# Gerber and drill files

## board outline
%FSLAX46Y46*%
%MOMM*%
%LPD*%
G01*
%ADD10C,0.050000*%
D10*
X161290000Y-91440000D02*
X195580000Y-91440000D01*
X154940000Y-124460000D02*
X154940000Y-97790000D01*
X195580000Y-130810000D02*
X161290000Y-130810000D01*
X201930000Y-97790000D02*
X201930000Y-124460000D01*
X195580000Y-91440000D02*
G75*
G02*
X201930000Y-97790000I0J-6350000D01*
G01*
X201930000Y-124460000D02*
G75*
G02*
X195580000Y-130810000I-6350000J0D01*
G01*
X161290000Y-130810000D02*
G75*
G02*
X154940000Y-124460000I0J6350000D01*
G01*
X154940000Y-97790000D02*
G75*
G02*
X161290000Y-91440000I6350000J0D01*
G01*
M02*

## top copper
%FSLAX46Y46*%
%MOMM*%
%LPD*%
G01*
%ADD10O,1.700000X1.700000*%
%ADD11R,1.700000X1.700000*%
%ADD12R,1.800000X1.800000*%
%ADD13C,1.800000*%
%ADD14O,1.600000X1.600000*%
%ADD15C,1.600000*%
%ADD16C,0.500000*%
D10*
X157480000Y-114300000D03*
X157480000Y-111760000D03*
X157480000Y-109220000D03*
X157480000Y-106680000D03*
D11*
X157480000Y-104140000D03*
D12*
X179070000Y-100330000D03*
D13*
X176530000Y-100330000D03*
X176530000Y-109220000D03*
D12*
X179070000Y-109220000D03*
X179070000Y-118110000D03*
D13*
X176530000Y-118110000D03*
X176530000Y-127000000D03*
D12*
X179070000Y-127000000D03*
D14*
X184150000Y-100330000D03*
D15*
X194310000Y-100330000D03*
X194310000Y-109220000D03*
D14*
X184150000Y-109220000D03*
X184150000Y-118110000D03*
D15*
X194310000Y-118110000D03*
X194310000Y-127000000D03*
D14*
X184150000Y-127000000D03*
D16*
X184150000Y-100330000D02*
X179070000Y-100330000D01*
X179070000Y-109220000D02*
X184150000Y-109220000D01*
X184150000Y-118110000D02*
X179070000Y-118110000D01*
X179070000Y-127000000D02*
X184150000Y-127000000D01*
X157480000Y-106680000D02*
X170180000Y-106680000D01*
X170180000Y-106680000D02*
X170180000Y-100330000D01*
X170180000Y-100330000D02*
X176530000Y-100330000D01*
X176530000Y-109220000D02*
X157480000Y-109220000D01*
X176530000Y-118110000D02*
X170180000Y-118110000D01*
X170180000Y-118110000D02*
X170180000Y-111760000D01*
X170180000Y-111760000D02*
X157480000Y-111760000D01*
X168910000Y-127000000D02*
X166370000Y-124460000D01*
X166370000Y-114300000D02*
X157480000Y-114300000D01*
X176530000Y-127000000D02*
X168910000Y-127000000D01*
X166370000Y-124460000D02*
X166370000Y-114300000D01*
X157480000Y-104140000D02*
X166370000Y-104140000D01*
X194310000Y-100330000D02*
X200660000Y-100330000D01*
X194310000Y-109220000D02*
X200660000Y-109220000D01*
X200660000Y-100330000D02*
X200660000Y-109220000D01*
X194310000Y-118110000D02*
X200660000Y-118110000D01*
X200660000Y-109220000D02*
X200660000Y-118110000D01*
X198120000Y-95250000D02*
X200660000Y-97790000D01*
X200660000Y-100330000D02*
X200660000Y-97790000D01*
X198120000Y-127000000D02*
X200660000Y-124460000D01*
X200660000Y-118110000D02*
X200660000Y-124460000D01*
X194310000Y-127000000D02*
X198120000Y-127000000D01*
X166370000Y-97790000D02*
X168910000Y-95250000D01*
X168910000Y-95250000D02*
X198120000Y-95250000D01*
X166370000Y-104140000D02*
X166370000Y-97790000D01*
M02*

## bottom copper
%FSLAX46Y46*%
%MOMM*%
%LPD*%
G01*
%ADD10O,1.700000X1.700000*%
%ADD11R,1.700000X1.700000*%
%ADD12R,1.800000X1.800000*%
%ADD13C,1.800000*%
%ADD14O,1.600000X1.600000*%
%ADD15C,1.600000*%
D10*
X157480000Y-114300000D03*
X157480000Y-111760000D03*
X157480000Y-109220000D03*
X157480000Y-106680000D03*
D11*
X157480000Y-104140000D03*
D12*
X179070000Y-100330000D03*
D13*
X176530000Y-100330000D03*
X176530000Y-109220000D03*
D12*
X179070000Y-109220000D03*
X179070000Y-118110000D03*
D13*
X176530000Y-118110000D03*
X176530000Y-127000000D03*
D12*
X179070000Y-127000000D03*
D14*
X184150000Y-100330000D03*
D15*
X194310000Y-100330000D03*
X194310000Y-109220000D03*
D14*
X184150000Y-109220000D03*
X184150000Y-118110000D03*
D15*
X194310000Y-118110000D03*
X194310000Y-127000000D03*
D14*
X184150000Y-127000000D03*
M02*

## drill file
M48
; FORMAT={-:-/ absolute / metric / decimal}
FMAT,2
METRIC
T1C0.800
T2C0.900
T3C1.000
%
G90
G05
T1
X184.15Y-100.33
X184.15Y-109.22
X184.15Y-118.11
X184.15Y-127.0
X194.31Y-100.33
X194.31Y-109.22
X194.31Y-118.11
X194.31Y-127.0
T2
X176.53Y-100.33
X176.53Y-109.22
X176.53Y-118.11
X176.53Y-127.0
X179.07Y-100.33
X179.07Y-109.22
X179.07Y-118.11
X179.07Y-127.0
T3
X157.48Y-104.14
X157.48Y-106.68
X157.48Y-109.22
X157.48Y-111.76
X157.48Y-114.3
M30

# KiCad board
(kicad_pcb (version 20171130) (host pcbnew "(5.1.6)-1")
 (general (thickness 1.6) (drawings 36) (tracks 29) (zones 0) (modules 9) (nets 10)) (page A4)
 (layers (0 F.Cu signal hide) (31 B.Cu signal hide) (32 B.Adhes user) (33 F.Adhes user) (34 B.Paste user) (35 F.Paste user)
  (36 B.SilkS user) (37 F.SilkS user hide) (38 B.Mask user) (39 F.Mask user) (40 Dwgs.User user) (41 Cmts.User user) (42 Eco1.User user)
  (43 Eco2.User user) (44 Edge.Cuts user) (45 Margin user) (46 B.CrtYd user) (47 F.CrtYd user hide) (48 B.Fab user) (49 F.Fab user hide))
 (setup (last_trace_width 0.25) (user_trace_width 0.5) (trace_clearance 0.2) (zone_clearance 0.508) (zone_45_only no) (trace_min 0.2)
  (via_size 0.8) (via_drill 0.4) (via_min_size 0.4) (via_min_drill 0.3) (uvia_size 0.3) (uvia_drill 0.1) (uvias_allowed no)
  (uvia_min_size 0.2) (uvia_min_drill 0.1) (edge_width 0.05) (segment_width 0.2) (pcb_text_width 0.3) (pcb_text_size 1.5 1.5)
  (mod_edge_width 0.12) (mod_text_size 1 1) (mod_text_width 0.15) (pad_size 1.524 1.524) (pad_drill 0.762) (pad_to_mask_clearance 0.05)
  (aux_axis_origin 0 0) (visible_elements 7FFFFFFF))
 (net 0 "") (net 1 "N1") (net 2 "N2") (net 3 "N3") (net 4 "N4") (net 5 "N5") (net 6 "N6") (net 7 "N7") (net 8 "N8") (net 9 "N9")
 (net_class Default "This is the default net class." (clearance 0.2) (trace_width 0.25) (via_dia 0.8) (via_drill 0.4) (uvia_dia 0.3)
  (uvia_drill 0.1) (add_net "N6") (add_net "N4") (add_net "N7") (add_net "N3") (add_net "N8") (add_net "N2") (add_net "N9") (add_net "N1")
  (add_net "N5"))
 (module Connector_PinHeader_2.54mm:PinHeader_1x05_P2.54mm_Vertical (layer F.Cu) (at 157.48 104.14)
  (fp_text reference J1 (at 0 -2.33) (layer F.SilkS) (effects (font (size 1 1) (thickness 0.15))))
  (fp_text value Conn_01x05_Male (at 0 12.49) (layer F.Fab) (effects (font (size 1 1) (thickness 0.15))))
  (pad 5 thru_hole oval (at 0 10.16) (size 1.7 1.7) (drill 1) (layers *.Cu *.Mask) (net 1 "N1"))
  (pad 4 thru_hole oval (at 0 7.62) (size 1.7 1.7) (drill 1) (layers *.Cu *.Mask) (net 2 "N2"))
  (pad 3 thru_hole oval (at 0 5.08) (size 1.7 1.7) (drill 1) (layers *.Cu *.Mask) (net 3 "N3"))
  (pad 2 thru_hole oval (at 0 2.54) (size 1.7 1.7) (drill 1) (layers *.Cu *.Mask) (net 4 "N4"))
  (pad 1 thru_hole rect (at 0 0) (size 1.7 1.7) (drill 1) (layers *.Cu *.Mask) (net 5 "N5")))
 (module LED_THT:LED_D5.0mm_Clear (layer F.Cu) (at 179.07 100.33 180)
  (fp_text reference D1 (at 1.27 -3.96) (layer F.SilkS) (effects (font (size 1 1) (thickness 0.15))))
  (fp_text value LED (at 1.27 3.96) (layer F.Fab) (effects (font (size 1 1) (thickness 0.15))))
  (pad 1 thru_hole rect (at 0 0 180) (size 1.8 1.8) (drill 0.9) (layers *.Cu *.Mask) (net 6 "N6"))
  (pad 2 thru_hole circle (at 2.54 0 180) (size 1.8 1.8) (drill 0.9) (layers *.Cu *.Mask) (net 4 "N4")))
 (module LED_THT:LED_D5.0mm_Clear (layer F.Cu) (at 179.07 109.22 180)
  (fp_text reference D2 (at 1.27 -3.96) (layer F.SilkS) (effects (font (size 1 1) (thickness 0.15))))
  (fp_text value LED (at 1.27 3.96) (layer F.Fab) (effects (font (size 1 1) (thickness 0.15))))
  (pad 2 thru_hole circle (at 2.54 0 180) (size 1.8 1.8) (drill 0.9) (layers *.Cu *.Mask) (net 3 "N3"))
  (pad 1 thru_hole rect (at 0 0 180) (size 1.8 1.8) (drill 0.9) (layers *.Cu *.Mask) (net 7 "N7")))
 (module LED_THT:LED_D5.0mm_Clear (layer F.Cu) (at 179.07 118.11 180)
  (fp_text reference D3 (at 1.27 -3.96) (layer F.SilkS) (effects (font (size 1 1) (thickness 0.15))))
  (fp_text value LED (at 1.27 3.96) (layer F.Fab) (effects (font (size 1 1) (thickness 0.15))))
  (pad 1 thru_hole rect (at 0 0 180) (size 1.8 1.8) (drill 0.9) (layers *.Cu *.Mask) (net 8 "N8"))
  (pad 2 thru_hole circle (at 2.54 0 180) (size 1.8 1.8) (drill 0.9) (layers *.Cu *.Mask) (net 2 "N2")))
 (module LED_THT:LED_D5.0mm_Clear (layer F.Cu) (at 179.07 127 180)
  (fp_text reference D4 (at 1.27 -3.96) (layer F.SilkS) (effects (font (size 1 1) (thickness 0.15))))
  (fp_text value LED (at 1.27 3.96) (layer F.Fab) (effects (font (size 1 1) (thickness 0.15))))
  (pad 2 thru_hole circle (at 2.54 0 180) (size 1.8 1.8) (drill 0.9) (layers *.Cu *.Mask) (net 1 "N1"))
  (pad 1 thru_hole rect (at 0 0 180) (size 1.8 1.8) (drill 0.9) (layers *.Cu *.Mask) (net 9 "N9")))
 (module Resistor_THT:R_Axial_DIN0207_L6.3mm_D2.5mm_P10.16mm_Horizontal (layer F.Cu) (at 194.31 100.33 180)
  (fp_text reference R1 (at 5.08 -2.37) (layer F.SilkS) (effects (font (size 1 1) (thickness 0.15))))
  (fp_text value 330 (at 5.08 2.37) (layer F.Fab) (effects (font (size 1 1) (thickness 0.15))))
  (pad 2 thru_hole oval (at 10.16 0 180) (size 1.6 1.6) (drill 0.8) (layers *.Cu *.Mask) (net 6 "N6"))
  (pad 1 thru_hole circle (at 0 0 180) (size 1.6 1.6) (drill 0.8) (layers *.Cu *.Mask) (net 5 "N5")))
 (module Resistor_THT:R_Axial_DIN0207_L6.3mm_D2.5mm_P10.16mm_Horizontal (layer F.Cu) (at 194.31 109.22 180)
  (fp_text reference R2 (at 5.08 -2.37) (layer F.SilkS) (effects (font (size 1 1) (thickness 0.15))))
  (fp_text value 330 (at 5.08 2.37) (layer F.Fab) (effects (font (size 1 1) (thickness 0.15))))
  (pad 1 thru_hole circle (at 0 0 180) (size 1.6 1.6) (drill 0.8) (layers *.Cu *.Mask) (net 5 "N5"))
  (pad 2 thru_hole oval (at 10.16 0 180) (size 1.6 1.6) (drill 0.8) (layers *.Cu *.Mask) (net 7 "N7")))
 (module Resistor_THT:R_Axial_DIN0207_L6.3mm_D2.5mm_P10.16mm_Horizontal (layer F.Cu) (at 194.31 118.11 180)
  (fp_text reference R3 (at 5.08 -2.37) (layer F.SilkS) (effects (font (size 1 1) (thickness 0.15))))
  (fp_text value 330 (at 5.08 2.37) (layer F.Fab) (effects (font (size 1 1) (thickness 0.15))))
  (pad 2 thru_hole oval (at 10.16 0 180) (size 1.6 1.6) (drill 0.8) (layers *.Cu *.Mask) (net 8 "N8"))
  (pad 1 thru_hole circle (at 0 0 180) (size 1.6 1.6) (drill 0.8) (layers *.Cu *.Mask) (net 5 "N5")))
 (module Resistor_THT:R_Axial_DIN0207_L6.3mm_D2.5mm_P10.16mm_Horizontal (layer F.Cu) (at 194.31 127 180)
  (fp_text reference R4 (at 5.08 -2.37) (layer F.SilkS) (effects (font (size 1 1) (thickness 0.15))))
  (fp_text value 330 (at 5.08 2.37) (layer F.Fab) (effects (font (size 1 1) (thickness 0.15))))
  (pad 1 thru_hole circle (at 0 0 180) (size 1.6 1.6) (drill 0.8) (layers *.Cu *.Mask) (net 5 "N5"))
  (pad 2 thru_hole oval (at 10.16 0 180) (size 1.6 1.6) (drill 0.8) (layers *.Cu *.Mask) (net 9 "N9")))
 (gr_line (start 161.29 91.44) (end 195.58 91.44) (layer Edge.Cuts) (width 0.05))
 (gr_line (start 154.94 124.46) (end 154.94 97.79) (layer Edge.Cuts) (width 0.05))
 (gr_line (start 195.58 130.81) (end 161.29 130.81) (layer Edge.Cuts) (width 0.05))
 (gr_line (start 201.93 97.79) (end 201.93 124.46) (layer Edge.Cuts) (width 0.05))
 (gr_arc (start 195.58 97.79) (end 201.93 97.79) (angle -90) (layer Edge.Cuts) (width 0.05))
 (gr_arc (start 195.58 124.46) (end 195.58 130.81) (angle -90) (layer Edge.Cuts) (width 0.05))
 (gr_arc (start 161.29 124.46) (end 154.94 124.46) (angle -90) (layer Edge.Cuts) (width 0.05))
 (gr_arc (start 161.29 97.79) (end 161.29 91.44) (angle -90) (layer Edge.Cuts) (width 0.05))
 (segment (start 184.15 100.33) (end 179.07 100.33) (width 0.5) (layer F.Cu) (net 6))
 (segment (start 179.07 109.22) (end 184.15 109.22) (width 0.5) (layer F.Cu) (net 7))
 (segment (start 184.15 118.11) (end 179.07 118.11) (width 0.5) (layer F.Cu) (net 8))
 (segment (start 179.07 127) (end 184.15 127) (width 0.5) (layer F.Cu) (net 9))
 (segment (start 157.48 106.68) (end 170.18 106.68) (width 0.5) (layer F.Cu) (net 4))
 (segment (start 170.18 106.68) (end 170.18 100.33) (width 0.5) (layer F.Cu) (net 4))
 (segment (start 170.18 100.33) (end 176.53 100.33) (width 0.5) (layer F.Cu) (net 4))
 (segment (start 176.53 109.22) (end 157.48 109.22) (width 0.5) (layer F.Cu) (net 3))
 (segment (start 176.53 118.11) (end 170.18 118.11) (width 0.5) (layer F.Cu) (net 2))
 (segment (start 170.18 118.11) (end 170.18 111.76) (width 0.5) (layer F.Cu) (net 2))
 (segment (start 170.18 111.76) (end 157.48 111.76) (width 0.5) (layer F.Cu) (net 2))
 (segment (start 168.91 127) (end 166.37 124.46) (width 0.5) (layer F.Cu) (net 1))
 (segment (start 166.37 114.3) (end 157.48 114.3) (width 0.5) (layer F.Cu) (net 1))
 (segment (start 176.53 127) (end 168.91 127) (width 0.5) (layer F.Cu) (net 1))
 (segment (start 166.37 124.46) (end 166.37 114.3) (width 0.5) (layer F.Cu) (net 1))
 (segment (start 157.48 104.14) (end 166.37 104.14) (width 0.5) (layer F.Cu) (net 5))
 (segment (start 194.31 100.33) (end 200.66 100.33) (width 0.5) (layer F.Cu) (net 5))
 (segment (start 194.31 109.22) (end 200.66 109.22) (width 0.5) (layer F.Cu) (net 5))
 (segment (start 200.66 100.33) (end 200.66 109.22) (width 0.5) (layer F.Cu) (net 5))
 (segment (start 194.31 118.11) (end 200.66 118.11) (width 0.5) (layer F.Cu) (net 5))
 (segment (start 200.66 109.22) (end 200.66 118.11) (width 0.5) (layer F.Cu) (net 5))
 (segment (start 198.12 95.25) (end 200.66 97.79) (width 0.5) (layer F.Cu) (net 5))
 (segment (start 200.66 100.33) (end 200.66 97.79) (width 0.5) (layer F.Cu) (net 5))
 (segment (start 198.12 127) (end 200.66 124.46) (width 0.5) (layer F.Cu) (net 5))
 (segment (start 200.66 118.11) (end 200.66 124.46) (width 0.5) (layer F.Cu) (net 5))
 (segment (start 194.31 127) (end 198.12 127) (width 0.5) (layer F.Cu) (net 5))
 (segment (start 166.37 97.79) (end 168.91 95.25) (width 0.5) (layer F.Cu) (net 5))
 (segment (start 168.91 95.25) (end 198.12 95.25) (width 0.5) (layer F.Cu) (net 5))
 (segment (start 166.37 104.14) (end 166.37 97.79) (width 0.5) (layer F.Cu) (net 5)))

